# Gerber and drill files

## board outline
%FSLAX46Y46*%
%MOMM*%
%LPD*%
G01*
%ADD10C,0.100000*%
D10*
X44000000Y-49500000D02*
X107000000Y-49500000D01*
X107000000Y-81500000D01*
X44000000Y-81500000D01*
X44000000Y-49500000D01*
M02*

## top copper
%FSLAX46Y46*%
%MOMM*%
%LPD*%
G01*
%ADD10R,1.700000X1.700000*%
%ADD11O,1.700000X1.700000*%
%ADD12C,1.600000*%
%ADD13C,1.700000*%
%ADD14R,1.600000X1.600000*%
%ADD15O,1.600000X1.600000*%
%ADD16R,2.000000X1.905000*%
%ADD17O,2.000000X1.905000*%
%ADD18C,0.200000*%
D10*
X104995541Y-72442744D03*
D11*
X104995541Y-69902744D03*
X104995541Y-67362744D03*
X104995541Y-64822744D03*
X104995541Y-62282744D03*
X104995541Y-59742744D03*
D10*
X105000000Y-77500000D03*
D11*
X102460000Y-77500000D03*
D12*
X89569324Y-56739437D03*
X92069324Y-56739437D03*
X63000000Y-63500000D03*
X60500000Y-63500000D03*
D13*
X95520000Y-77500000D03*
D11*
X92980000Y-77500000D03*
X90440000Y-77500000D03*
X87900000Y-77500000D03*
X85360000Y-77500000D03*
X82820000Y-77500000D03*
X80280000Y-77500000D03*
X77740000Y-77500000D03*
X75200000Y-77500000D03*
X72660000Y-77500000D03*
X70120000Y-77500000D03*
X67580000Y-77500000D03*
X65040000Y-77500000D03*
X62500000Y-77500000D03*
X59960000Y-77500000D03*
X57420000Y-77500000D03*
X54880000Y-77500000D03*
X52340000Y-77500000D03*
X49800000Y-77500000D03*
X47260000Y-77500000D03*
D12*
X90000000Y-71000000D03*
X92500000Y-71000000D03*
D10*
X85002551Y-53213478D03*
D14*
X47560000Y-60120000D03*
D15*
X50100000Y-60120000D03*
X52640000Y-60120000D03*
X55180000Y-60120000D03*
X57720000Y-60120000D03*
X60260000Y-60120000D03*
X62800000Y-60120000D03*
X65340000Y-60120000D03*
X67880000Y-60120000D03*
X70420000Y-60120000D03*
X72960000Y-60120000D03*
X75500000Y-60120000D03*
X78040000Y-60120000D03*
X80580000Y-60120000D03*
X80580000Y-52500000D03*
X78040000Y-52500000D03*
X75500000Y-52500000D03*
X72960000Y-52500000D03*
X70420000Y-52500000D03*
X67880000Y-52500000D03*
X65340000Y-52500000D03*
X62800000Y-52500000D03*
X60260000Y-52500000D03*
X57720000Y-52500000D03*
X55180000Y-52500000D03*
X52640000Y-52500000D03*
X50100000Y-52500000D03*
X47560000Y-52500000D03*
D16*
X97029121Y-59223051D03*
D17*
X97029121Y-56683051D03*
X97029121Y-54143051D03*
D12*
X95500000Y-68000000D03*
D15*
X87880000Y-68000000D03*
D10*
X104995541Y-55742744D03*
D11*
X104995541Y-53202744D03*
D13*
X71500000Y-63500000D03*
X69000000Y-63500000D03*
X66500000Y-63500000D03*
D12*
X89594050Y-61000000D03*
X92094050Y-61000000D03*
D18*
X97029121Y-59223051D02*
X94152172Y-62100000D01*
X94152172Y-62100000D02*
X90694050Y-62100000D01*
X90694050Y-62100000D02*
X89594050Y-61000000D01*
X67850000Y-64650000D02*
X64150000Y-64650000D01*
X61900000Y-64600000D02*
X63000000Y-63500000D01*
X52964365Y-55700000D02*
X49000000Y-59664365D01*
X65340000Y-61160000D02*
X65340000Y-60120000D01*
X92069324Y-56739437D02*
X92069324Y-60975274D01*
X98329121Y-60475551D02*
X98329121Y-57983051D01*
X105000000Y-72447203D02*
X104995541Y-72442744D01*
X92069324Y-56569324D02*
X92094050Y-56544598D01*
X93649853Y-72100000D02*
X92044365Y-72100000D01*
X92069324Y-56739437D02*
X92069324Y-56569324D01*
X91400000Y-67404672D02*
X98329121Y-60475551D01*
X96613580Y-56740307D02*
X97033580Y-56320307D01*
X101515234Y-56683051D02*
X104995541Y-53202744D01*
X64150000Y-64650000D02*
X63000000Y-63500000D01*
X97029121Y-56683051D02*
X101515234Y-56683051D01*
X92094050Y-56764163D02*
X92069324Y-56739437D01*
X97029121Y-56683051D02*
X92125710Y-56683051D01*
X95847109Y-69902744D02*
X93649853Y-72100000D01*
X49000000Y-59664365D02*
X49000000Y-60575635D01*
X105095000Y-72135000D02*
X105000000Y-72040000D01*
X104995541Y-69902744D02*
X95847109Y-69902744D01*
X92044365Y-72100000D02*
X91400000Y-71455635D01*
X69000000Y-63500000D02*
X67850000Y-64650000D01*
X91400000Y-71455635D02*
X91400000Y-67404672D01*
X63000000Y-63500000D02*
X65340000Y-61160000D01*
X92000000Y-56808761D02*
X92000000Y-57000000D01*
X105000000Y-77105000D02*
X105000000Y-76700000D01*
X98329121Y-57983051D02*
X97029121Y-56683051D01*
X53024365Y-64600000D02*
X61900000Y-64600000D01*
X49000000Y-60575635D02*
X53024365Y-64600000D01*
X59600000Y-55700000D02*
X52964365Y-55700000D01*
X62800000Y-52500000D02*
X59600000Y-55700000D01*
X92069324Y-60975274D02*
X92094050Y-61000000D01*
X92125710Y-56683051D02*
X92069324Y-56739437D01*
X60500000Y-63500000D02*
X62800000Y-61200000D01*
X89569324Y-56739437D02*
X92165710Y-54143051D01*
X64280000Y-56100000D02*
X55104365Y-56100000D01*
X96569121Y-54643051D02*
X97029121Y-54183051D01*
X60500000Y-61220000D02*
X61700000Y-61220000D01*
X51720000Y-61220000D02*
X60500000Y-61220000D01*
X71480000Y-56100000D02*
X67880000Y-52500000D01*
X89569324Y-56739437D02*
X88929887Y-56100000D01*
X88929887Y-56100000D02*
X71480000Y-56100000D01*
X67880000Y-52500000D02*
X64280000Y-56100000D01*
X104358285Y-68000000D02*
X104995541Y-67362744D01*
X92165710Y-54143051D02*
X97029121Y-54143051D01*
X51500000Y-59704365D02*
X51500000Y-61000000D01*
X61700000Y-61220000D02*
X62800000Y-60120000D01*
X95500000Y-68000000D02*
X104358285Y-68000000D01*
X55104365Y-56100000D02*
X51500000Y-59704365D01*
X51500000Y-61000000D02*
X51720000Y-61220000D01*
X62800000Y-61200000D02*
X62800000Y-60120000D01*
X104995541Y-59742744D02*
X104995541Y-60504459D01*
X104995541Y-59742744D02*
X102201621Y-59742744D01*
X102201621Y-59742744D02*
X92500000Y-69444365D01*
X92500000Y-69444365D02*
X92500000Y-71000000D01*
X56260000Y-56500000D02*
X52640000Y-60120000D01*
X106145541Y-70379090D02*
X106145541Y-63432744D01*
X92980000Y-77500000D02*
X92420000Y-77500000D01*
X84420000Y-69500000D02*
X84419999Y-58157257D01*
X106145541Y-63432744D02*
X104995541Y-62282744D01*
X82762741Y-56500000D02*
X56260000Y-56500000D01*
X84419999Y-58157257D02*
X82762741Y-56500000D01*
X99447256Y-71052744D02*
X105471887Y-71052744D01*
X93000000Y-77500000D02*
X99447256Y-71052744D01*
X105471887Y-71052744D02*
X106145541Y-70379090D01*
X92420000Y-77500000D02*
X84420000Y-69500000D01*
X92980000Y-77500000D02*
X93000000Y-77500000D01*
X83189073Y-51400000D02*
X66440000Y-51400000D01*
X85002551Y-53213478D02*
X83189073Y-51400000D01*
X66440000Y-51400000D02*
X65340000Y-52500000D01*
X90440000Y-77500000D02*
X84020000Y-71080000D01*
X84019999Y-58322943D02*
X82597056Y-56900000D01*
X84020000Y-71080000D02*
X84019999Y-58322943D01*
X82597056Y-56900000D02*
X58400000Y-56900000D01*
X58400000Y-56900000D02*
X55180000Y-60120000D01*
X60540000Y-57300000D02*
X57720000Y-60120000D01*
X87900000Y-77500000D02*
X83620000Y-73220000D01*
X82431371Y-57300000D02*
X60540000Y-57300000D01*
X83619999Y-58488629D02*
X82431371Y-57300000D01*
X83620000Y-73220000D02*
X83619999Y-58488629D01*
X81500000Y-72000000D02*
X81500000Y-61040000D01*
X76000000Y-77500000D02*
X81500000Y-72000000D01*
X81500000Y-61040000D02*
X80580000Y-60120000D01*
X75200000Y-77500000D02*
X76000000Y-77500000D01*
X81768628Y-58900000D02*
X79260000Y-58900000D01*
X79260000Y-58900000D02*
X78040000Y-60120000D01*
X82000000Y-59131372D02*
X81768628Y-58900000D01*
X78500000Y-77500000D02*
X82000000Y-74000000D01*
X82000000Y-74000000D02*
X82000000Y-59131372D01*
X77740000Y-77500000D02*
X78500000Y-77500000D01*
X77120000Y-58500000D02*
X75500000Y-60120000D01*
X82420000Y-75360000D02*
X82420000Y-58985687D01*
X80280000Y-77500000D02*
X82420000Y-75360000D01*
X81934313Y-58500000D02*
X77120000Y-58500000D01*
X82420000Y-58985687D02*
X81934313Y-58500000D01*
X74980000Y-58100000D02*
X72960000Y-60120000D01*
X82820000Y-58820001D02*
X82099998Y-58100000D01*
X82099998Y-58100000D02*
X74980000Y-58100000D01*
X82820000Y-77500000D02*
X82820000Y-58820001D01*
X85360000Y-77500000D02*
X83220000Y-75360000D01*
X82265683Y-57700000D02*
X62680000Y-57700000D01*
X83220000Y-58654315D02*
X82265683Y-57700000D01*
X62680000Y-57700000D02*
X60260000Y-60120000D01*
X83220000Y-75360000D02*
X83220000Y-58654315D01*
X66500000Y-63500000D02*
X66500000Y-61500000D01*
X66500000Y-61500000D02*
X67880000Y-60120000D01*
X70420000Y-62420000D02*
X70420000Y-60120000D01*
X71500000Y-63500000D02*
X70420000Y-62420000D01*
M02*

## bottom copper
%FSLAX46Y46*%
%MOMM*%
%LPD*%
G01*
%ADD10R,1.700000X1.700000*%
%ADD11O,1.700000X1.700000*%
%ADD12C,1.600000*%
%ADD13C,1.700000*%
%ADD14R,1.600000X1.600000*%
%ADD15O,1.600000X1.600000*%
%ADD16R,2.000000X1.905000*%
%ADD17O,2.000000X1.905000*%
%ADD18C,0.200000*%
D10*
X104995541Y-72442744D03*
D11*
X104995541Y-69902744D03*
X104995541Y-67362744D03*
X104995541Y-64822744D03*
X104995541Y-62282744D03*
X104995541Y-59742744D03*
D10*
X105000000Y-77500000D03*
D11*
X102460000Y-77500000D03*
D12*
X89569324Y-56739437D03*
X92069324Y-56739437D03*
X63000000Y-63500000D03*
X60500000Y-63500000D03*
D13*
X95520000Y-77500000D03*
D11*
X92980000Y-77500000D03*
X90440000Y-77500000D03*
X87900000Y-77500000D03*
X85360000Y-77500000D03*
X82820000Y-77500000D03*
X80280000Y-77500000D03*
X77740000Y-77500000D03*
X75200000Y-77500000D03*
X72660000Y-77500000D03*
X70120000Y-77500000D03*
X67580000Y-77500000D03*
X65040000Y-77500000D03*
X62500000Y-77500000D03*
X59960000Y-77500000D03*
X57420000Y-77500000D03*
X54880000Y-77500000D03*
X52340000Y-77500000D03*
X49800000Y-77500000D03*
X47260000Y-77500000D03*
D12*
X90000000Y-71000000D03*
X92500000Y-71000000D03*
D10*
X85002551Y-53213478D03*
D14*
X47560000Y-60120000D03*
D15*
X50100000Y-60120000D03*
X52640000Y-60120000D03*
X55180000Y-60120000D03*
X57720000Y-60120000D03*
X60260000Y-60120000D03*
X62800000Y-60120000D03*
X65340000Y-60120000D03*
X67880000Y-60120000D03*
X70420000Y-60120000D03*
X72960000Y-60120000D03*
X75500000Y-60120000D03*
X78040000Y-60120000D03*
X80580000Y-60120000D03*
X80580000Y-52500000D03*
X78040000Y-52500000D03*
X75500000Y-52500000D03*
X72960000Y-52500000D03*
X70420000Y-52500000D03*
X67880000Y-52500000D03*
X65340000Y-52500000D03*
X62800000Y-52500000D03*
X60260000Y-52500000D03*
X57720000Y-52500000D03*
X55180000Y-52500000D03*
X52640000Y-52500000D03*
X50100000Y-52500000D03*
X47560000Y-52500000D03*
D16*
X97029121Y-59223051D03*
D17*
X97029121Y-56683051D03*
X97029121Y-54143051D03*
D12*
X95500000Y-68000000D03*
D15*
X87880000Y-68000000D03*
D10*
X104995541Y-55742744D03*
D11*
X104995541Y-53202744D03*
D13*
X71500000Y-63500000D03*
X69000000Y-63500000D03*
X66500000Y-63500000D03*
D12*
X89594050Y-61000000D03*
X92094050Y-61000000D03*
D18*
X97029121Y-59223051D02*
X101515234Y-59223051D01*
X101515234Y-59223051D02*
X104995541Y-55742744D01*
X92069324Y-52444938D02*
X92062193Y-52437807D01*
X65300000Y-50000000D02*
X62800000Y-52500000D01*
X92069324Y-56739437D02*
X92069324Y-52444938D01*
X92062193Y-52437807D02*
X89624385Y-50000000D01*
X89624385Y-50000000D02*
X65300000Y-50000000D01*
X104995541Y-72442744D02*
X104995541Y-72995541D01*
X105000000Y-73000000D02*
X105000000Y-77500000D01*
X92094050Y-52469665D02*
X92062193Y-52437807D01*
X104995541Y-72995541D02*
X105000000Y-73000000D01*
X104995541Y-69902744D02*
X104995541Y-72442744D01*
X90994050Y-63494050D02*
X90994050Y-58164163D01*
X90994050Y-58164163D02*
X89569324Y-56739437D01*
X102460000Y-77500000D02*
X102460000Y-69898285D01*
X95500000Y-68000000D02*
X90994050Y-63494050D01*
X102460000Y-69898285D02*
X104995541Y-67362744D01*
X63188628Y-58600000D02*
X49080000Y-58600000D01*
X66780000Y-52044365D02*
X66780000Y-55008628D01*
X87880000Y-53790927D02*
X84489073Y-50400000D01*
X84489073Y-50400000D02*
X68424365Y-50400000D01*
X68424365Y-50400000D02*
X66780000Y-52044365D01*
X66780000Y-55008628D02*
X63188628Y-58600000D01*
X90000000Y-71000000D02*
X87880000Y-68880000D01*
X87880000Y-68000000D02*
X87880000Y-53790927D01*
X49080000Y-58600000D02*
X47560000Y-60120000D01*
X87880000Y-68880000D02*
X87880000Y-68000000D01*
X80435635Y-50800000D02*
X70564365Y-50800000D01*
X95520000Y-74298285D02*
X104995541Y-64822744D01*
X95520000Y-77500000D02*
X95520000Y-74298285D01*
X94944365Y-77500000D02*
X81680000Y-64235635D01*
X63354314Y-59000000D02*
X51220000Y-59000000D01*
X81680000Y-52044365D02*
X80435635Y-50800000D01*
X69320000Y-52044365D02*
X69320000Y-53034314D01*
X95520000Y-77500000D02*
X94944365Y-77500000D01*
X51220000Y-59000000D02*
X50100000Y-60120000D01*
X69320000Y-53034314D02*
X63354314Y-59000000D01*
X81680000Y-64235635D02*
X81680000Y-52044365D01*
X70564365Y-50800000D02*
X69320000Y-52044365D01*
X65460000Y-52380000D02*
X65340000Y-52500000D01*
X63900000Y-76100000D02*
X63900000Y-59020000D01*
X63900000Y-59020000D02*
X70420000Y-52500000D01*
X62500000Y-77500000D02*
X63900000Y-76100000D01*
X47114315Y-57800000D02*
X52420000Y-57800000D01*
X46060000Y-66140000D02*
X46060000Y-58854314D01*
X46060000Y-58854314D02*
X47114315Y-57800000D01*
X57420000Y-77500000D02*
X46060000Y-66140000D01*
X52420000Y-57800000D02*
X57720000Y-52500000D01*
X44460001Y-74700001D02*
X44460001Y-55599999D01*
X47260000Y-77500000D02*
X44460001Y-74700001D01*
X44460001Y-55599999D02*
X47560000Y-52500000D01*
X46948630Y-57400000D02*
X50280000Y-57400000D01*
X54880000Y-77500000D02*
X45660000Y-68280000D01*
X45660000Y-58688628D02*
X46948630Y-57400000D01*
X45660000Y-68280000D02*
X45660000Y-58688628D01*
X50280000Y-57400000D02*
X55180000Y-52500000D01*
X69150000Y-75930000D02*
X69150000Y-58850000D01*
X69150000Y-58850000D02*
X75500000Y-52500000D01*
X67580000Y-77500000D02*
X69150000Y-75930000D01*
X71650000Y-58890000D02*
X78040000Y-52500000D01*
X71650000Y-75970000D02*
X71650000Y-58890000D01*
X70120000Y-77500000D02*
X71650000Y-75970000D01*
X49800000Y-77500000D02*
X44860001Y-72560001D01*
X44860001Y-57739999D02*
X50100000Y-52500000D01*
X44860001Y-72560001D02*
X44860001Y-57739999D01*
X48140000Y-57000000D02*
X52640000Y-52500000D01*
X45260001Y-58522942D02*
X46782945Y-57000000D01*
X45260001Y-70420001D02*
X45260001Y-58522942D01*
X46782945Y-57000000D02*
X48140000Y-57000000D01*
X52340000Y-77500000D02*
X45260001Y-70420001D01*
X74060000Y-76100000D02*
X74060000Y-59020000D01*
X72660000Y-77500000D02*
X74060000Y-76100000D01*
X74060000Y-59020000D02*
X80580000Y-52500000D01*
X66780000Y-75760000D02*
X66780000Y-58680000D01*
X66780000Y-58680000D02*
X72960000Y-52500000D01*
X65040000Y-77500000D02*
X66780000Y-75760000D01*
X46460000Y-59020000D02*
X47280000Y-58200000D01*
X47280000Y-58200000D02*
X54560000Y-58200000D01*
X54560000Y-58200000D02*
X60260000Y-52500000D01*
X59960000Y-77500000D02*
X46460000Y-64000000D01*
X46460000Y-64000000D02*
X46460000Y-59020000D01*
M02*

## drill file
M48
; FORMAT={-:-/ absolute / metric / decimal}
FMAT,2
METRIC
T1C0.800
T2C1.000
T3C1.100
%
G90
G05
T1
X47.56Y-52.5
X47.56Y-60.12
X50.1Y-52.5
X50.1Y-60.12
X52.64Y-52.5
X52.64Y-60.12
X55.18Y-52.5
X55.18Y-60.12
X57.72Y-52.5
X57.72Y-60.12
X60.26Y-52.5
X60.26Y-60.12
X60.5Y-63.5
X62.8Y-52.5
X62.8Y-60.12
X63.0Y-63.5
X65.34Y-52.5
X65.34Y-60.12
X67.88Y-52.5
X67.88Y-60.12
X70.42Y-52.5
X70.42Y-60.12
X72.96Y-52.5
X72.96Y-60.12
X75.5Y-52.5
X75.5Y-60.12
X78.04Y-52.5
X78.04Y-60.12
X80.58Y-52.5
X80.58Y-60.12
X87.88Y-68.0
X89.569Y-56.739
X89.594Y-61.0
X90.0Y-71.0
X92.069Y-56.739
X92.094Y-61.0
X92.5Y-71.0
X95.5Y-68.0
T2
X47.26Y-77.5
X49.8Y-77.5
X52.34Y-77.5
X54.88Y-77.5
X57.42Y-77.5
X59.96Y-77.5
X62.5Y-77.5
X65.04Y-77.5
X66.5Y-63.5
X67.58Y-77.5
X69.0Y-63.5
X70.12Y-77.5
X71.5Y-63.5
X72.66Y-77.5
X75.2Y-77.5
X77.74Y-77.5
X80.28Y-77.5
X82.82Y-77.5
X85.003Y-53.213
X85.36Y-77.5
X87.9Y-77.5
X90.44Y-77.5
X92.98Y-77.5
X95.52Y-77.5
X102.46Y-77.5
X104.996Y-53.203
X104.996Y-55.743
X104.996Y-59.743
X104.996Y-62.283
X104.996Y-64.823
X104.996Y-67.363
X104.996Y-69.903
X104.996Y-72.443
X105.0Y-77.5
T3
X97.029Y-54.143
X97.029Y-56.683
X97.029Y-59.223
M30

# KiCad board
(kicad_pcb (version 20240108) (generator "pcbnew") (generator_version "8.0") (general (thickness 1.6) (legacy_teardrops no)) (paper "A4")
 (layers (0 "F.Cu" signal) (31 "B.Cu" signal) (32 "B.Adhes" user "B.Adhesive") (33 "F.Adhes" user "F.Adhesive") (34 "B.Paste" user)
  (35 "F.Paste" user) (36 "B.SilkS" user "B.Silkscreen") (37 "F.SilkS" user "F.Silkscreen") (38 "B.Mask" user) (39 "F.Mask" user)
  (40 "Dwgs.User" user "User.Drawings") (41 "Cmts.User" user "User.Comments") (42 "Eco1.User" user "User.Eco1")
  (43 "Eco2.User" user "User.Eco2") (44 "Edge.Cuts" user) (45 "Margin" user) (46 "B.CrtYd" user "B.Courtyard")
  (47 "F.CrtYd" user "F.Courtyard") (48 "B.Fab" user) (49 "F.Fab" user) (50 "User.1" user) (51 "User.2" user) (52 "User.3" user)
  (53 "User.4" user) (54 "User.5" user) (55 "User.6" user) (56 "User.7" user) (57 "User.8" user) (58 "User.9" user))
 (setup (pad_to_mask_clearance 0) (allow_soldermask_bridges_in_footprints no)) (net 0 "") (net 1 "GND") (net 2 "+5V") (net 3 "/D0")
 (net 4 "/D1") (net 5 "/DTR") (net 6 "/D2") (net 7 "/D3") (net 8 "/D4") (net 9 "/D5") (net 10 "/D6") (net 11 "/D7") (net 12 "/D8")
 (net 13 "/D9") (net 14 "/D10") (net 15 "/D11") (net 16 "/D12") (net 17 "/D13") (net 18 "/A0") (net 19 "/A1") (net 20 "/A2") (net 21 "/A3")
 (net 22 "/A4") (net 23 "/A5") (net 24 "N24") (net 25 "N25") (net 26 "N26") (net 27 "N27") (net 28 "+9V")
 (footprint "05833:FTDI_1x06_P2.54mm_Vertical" (layer "F.Cu") (at 104.995541 72.442744 180)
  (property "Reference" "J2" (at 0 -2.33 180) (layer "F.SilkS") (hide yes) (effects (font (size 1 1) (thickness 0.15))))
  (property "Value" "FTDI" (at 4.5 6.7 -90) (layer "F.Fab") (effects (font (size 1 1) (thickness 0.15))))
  (pad "1" thru_hole rect (at 0 0 180) (size 1.7 1.7) (drill 1) (layers "*.Cu" "*.Mask") (remove_unused_layers no) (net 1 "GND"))
  (pad "2" thru_hole oval (at 0 2.54 180) (size 1.7 1.7) (drill 1) (layers "*.Cu" "*.Mask") (remove_unused_layers no) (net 1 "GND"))
  (pad "3" thru_hole oval (at 0 5.08 180) (size 1.7 1.7) (drill 1) (layers "*.Cu" "*.Mask") (remove_unused_layers no) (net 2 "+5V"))
  (pad "4" thru_hole oval (at 0 7.62 180) (size 1.7 1.7) (drill 1) (layers "*.Cu" "*.Mask") (remove_unused_layers no) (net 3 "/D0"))
  (pad "5" thru_hole oval (at 0 10.16 180) (size 1.7 1.7) (drill 1) (layers "*.Cu" "*.Mask") (remove_unused_layers no) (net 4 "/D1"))
  (pad "6" thru_hole oval (at 0 12.7 180) (size 1.7 1.7) (drill 1) (layers "*.Cu" "*.Mask") (remove_unused_layers no) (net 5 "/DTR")))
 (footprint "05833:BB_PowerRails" (layer "F.Cu") (at 105 77.5 -90)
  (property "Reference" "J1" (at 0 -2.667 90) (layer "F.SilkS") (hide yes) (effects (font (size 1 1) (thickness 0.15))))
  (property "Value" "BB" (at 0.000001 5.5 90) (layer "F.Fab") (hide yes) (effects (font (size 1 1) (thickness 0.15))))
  (pad "1" thru_hole rect (at 0 0 270) (size 1.7 1.7) (drill 1) (layers "*.Cu" "*.Mask") (remove_unused_layers no) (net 1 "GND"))
  (pad "2" thru_hole oval (at 0 2.54 270) (size 1.7 1.7) (drill 1) (layers "*.Cu" "*.Mask") (remove_unused_layers no) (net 2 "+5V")))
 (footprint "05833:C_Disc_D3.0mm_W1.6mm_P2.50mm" (layer "F.Cu") (at 89.569324 56.739437)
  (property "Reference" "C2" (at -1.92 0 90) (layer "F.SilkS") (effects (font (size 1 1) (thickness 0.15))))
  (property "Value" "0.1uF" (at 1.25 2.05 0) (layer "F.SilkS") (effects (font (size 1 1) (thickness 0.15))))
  (pad "1" thru_hole circle (at 0 0) (size 1.6 1.6) (drill 0.8) (layers "*.Cu" "*.Mask") (remove_unused_layers no) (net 2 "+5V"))
  (pad "2" thru_hole circle (at 2.5 0) (size 1.6 1.6) (drill 0.8) (layers "*.Cu" "*.Mask") (remove_unused_layers no) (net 1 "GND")))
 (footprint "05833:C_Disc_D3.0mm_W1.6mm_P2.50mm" (layer "F.Cu") (at 63 63.5 180)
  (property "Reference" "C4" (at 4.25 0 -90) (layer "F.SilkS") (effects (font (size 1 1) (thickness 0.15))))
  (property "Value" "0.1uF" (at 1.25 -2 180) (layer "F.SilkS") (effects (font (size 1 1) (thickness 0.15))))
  (pad "1" thru_hole circle (at 0 0 180) (size 1.6 1.6) (drill 0.8) (layers "*.Cu" "*.Mask") (remove_unused_layers no) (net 1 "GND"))
  (pad "2" thru_hole circle (at 2.5 0 180) (size 1.6 1.6) (drill 0.8) (layers "*.Cu" "*.Mask") (remove_unused_layers no) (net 2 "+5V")))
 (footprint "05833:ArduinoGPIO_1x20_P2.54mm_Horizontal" (layer "F.Cu") (at 95.52 77.5 -90)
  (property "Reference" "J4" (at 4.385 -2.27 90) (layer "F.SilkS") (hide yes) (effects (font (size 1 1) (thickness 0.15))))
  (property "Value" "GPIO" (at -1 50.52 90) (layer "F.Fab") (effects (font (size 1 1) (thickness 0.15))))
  (pad "1" thru_hole circle (at 0 0 270) (size 1.7 1.7) (drill 1) (layers "*.Cu" "*.Mask") (remove_unused_layers no) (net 3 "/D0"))
  (pad "2" thru_hole oval (at 0 2.54 270) (size 1.7 1.7) (drill 1) (layers "*.Cu" "*.Mask") (remove_unused_layers no) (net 4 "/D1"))
  (pad "3" thru_hole oval (at 0 5.08 270) (size 1.7 1.7) (drill 1) (layers "*.Cu" "*.Mask") (remove_unused_layers no) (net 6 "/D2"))
  (pad "4" thru_hole oval (at 0 7.62 270) (size 1.7 1.7) (drill 1) (layers "*.Cu" "*.Mask") (remove_unused_layers no) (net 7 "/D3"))
  (pad "5" thru_hole oval (at 0 10.16 270) (size 1.7 1.7) (drill 1) (layers "*.Cu" "*.Mask") (remove_unused_layers no) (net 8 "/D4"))
  (pad "6" thru_hole oval (at 0 12.7 270) (size 1.7 1.7) (drill 1) (layers "*.Cu" "*.Mask") (remove_unused_layers no) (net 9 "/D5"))
  (pad "7" thru_hole oval (at 0 15.24 270) (size 1.7 1.7) (drill 1) (layers "*.Cu" "*.Mask") (remove_unused_layers no) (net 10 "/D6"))
  (pad "8" thru_hole oval (at 0 17.78 270) (size 1.7 1.7) (drill 1) (layers "*.Cu" "*.Mask") (remove_unused_layers no) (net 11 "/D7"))
  (pad "9" thru_hole oval (at 0 20.32 270) (size 1.7 1.7) (drill 1) (layers "*.Cu" "*.Mask") (remove_unused_layers no) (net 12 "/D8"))
  (pad "10" thru_hole oval (at 0 22.86 270) (size 1.7 1.7) (drill 1) (layers "*.Cu" "*.Mask") (remove_unused_layers no) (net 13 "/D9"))
  (pad "11" thru_hole oval (at 0 25.4 270) (size 1.7 1.7) (drill 1) (layers "*.Cu" "*.Mask") (remove_unused_layers no) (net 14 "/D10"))
  (pad "12" thru_hole oval (at 0 27.94 270) (size 1.7 1.7) (drill 1) (layers "*.Cu" "*.Mask") (remove_unused_layers no) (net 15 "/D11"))
  (pad "13" thru_hole oval (at 0 30.48 270) (size 1.7 1.7) (drill 1) (layers "*.Cu" "*.Mask") (remove_unused_layers no) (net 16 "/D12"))
  (pad "14" thru_hole oval (at 0 33.02 270) (size 1.7 1.7) (drill 1) (layers "*.Cu" "*.Mask") (remove_unused_layers no) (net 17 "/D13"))
  (pad "15" thru_hole oval (at 0 35.56 270) (size 1.7 1.7) (drill 1) (layers "*.Cu" "*.Mask") (remove_unused_layers no) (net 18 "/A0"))
  (pad "16" thru_hole oval (at 0 38.1 270) (size 1.7 1.7) (drill 1) (layers "*.Cu" "*.Mask") (remove_unused_layers no) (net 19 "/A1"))
  (pad "17" thru_hole oval (at 0 40.64 270) (size 1.7 1.7) (drill 1) (layers "*.Cu" "*.Mask") (remove_unused_layers no) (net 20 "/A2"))
  (pad "18" thru_hole oval (at 0 43.18 270) (size 1.7 1.7) (drill 1) (layers "*.Cu" "*.Mask") (remove_unused_layers no) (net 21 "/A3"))
  (pad "19" thru_hole oval (at 0 45.72 270) (size 1.7 1.7) (drill 1) (layers "*.Cu" "*.Mask") (remove_unused_layers no) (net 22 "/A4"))
  (pad "20" thru_hole oval (at 0 48.26 270) (size 1.7 1.7) (drill 1) (layers "*.Cu" "*.Mask") (remove_unused_layers no) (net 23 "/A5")))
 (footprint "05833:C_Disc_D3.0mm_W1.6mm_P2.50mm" (layer "F.Cu") (at 90 71)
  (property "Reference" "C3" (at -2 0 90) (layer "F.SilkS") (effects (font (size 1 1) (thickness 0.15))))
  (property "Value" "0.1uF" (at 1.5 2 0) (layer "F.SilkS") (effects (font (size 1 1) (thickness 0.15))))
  (pad "1" thru_hole circle (at 0 0) (size 1.6 1.6) (drill 0.8) (layers "*.Cu" "*.Mask") (remove_unused_layers no) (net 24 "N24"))
  (pad "2" thru_hole circle (at 2.5 0) (size 1.6 1.6) (drill 0.8) (layers "*.Cu" "*.Mask") (remove_unused_layers no) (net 5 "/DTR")))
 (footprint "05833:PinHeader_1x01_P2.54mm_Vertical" (layer "F.Cu") (at 85.002551 53.213478)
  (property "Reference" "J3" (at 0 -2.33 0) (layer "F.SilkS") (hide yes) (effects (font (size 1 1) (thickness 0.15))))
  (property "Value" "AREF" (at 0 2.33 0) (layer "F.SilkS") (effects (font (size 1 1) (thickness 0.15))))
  (pad "1" thru_hole rect (at 0 0) (size 1.7 1.7) (drill 1) (layers "*.Cu" "*.Mask") (remove_unused_layers no) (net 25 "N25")))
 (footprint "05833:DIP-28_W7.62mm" (layer "F.Cu") (at 47.56 60.12 90)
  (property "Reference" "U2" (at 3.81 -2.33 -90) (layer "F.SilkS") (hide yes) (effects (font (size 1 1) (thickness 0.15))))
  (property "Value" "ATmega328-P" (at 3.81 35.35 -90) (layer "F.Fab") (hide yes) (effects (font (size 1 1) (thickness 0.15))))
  (pad "1" thru_hole rect (at 0 0 90) (size 1.6 1.6) (drill 0.8) (layers "*.Cu" "*.Mask") (remove_unused_layers no) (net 24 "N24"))
  (pad "2" thru_hole oval (at 0 2.54 90) (size 1.6 1.6) (drill 0.8) (layers "*.Cu" "*.Mask") (remove_unused_layers no) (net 3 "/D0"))
  (pad "3" thru_hole oval (at 0 5.08 90) (size 1.6 1.6) (drill 0.8) (layers "*.Cu" "*.Mask") (remove_unused_layers no) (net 4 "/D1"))
  (pad "4" thru_hole oval (at 0 7.62 90) (size 1.6 1.6) (drill 0.8) (layers "*.Cu" "*.Mask") (remove_unused_layers no) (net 6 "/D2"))
  (pad "5" thru_hole oval (at 0 10.16 90) (size 1.6 1.6) (drill 0.8) (layers "*.Cu" "*.Mask") (remove_unused_layers no) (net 7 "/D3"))
  (pad "6" thru_hole oval (at 0 12.7 90) (size 1.6 1.6) (drill 0.8) (layers "*.Cu" "*.Mask") (remove_unused_layers no) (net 8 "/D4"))
  (pad "7" thru_hole oval (at 0 15.24 90) (size 1.6 1.6) (drill 0.8) (layers "*.Cu" "*.Mask") (remove_unused_layers no) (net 2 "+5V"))
  (pad "8" thru_hole oval (at 0 17.78 90) (size 1.6 1.6) (drill 0.8) (layers "*.Cu" "*.Mask") (remove_unused_layers no) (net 1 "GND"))
  (pad "9" thru_hole oval (at 0 20.32 90) (size 1.6 1.6) (drill 0.8) (layers "*.Cu" "*.Mask") (remove_unused_layers no) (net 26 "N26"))
  (pad "10" thru_hole oval (at 0 22.86 90) (size 1.6 1.6) (drill 0.8) (layers "*.Cu" "*.Mask") (remove_unused_layers no) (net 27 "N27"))
  (pad "11" thru_hole oval (at 0 25.4 90) (size 1.6 1.6) (drill 0.8) (layers "*.Cu" "*.Mask") (remove_unused_layers no) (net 9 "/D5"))
  (pad "12" thru_hole oval (at 0 27.94 90) (size 1.6 1.6) (drill 0.8) (layers "*.Cu" "*.Mask") (remove_unused_layers no) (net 10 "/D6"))
  (pad "13" thru_hole oval (at 0 30.48 90) (size 1.6 1.6) (drill 0.8) (layers "*.Cu" "*.Mask") (remove_unused_layers no) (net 11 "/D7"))
  (pad "14" thru_hole oval (at 0 33.02 90) (size 1.6 1.6) (drill 0.8) (layers "*.Cu" "*.Mask") (remove_unused_layers no) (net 12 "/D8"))
  (pad "15" thru_hole oval (at 7.62 33.02 90) (size 1.6 1.6) (drill 0.8) (layers "*.Cu" "*.Mask") (remove_unused_layers no) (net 13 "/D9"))
  (pad "16" thru_hole oval (at 7.62 30.48 90) (size 1.6 1.6) (drill 0.8) (layers "*.Cu" "*.Mask") (remove_unused_layers no) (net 14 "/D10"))
  (pad "17" thru_hole oval (at 7.62 27.94 90) (size 1.6 1.6) (drill 0.8) (layers "*.Cu" "*.Mask") (remove_unused_layers no) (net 15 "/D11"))
  (pad "18" thru_hole oval (at 7.62 25.4 90) (size 1.6 1.6) (drill 0.8) (layers "*.Cu" "*.Mask") (remove_unused_layers no) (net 16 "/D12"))
  (pad "19" thru_hole oval (at 7.62 22.86 90) (size 1.6 1.6) (drill 0.8) (layers "*.Cu" "*.Mask") (remove_unused_layers no) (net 17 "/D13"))
  (pad "20" thru_hole oval (at 7.62 20.32 90) (size 1.6 1.6) (drill 0.8) (layers "*.Cu" "*.Mask") (remove_unused_layers no) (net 2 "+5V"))
  (pad "21" thru_hole oval (at 7.62 17.78 90) (size 1.6 1.6) (drill 0.8) (layers "*.Cu" "*.Mask") (remove_unused_layers no) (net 25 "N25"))
  (pad "22" thru_hole oval (at 7.62 15.24 90) (size 1.6 1.6) (drill 0.8) (layers "*.Cu" "*.Mask") (remove_unused_layers no) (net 1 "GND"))
  (pad "23" thru_hole oval (at 7.62 12.7 90) (size 1.6 1.6) (drill 0.8) (layers "*.Cu" "*.Mask") (remove_unused_layers no) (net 18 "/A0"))
  (pad "24" thru_hole oval (at 7.62 10.16 90) (size 1.6 1.6) (drill 0.8) (layers "*.Cu" "*.Mask") (remove_unused_layers no) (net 19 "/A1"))
  (pad "25" thru_hole oval (at 7.62 7.62 90) (size 1.6 1.6) (drill 0.8) (layers "*.Cu" "*.Mask") (remove_unused_layers no) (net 20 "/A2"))
  (pad "26" thru_hole oval (at 7.62 5.08 90) (size 1.6 1.6) (drill 0.8) (layers "*.Cu" "*.Mask") (remove_unused_layers no) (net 21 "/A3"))
  (pad "27" thru_hole oval (at 7.62 2.54 90) (size 1.6 1.6) (drill 0.8) (layers "*.Cu" "*.Mask") (remove_unused_layers no) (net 22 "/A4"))
  (pad "28" thru_hole oval (at 7.62 0 90) (size 1.6 1.6) (drill 0.8) (layers "*.Cu" "*.Mask") (remove_unused_layers no) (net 23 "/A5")))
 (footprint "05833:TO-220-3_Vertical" (layer "F.Cu") (at 97.029121 59.223051 90)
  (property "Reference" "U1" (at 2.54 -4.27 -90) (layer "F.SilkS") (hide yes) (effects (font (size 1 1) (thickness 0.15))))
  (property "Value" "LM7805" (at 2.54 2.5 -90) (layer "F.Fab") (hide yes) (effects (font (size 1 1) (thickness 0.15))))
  (pad "1" thru_hole rect (at 0 0 90) (size 1.905 2) (drill 1.1) (layers "*.Cu" "*.Mask") (remove_unused_layers no) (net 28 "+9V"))
  (pad "2" thru_hole oval (at 2.54 0 90) (size 1.905 2) (drill 1.1) (layers "*.Cu" "*.Mask") (remove_unused_layers no) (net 1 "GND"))
  (pad "3" thru_hole oval (at 5.08 0 90) (size 1.905 2) (drill 1.1) (layers "*.Cu" "*.Mask") (remove_unused_layers no) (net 2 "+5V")))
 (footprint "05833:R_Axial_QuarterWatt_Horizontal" (layer "F.Cu") (at 95.5 68 180)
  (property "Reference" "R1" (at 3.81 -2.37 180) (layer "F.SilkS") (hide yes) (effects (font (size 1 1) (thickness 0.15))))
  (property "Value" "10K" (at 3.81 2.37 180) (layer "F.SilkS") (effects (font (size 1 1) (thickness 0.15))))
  (pad "1" thru_hole circle (at 0 0 180) (size 1.6 1.6) (drill 0.8) (layers "*.Cu" "*.Mask") (remove_unused_layers no) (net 2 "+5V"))
  (pad "2" thru_hole oval (at 7.62 0 180) (size 1.6 1.6) (drill 0.8) (layers "*.Cu" "*.Mask") (remove_unused_layers no) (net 24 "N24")))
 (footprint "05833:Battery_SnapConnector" (layer "F.Cu") (at 104.995541 55.742744 180)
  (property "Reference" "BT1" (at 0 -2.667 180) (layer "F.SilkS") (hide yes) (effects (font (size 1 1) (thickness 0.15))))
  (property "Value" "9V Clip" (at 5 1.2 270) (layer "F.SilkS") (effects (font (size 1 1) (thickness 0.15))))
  (pad "1" thru_hole rect (at 0 0 180) (size 1.7 1.7) (drill 1) (layers "*.Cu" "*.Mask") (remove_unused_layers no) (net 28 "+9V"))
  (pad "2" thru_hole oval (at 0 2.54 180) (size 1.7 1.7) (drill 1) (layers "*.Cu" "*.Mask") (remove_unused_layers no) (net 1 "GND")))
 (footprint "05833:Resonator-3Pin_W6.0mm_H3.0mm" (layer "F.Cu") (at 71.5 63.5 180)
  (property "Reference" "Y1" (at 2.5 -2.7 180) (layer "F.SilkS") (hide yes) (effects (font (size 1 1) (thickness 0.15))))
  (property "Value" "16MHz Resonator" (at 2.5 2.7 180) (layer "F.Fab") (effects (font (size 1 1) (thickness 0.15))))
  (pad "1" thru_hole circle (at 0 0 180) (size 1.7 1.7) (drill 1) (layers "*.Cu" "*.Mask") (remove_unused_layers no) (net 27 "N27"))
  (pad "2" thru_hole circle (at 2.5 0 180) (size 1.7 1.7) (drill 1) (layers "*.Cu" "*.Mask") (remove_unused_layers no) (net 1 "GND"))
  (pad "3" thru_hole circle (at 5 0 180) (size 1.7 1.7) (drill 1) (layers "*.Cu" "*.Mask") (remove_unused_layers no) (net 26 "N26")))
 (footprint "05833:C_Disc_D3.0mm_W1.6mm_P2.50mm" (layer "F.Cu") (at 89.59405 61)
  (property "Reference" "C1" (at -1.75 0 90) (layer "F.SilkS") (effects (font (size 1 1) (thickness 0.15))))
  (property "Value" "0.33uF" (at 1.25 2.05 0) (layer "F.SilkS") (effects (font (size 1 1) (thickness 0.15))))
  (pad "1" thru_hole circle (at 0 0) (size 1.6 1.6) (drill 0.8) (layers "*.Cu" "*.Mask") (remove_unused_layers no) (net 28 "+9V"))
  (pad "2" thru_hole circle (at 2.5 0) (size 1.6 1.6) (drill 0.8) (layers "*.Cu" "*.Mask") (remove_unused_layers no) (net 1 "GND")))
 (gr_rect (start 44 49.5) (end 107 81.5) (stroke (width 0.1) (type default)) (fill none) (layer "Edge.Cuts"))
 (segment (start 97.029121 59.223051) (end 94.152172 62.1) (width 0.2) (layer "F.Cu") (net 28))
 (segment (start 94.152172 62.1) (end 90.69405 62.1) (width 0.2) (layer "F.Cu") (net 28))
 (segment (start 90.69405 62.1) (end 89.59405 61) (width 0.2) (layer "F.Cu") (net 28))
 (segment (start 97.029121 59.223051) (end 101.515234 59.223051) (width 0.2) (layer "B.Cu") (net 28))
 (segment (start 101.515234 59.223051) (end 104.995541 55.742744) (width 0.2) (layer "B.Cu") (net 28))
 (segment (start 67.85 64.65) (end 64.15 64.65) (width 0.2) (layer "F.Cu") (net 1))
 (segment (start 61.9 64.6) (end 63 63.5) (width 0.2) (layer "F.Cu") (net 1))
 (segment (start 52.964365 55.7) (end 49 59.664365) (width 0.2) (layer "F.Cu") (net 1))
 (segment (start 65.34 61.16) (end 65.34 60.12) (width 0.2) (layer "F.Cu") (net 1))
 (segment (start 92.069324 56.739437) (end 92.069324 60.975274) (width 0.2) (layer "F.Cu") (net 1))
 (segment (start 98.329121 60.475551) (end 98.329121 57.983051) (width 0.2) (layer "F.Cu") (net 1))
 (segment (start 105 72.447203) (end 104.995541 72.442744) (width 0.2) (layer "F.Cu") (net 1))
 (segment (start 92.069324 56.569324) (end 92.09405 56.544598) (width 0.2) (layer "F.Cu") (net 1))
 (segment (start 93.649853 72.1) (end 92.044365 72.1) (width 0.2) (layer "F.Cu") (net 1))
 (segment (start 92.069324 56.739437) (end 92.069324 56.569324) (width 0.2) (layer "F.Cu") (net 1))
 (segment (start 91.4 67.404672) (end 98.329121 60.475551) (width 0.2) (layer "F.Cu") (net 1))
 (segment (start 96.61358 56.740307) (end 97.03358 56.320307) (width 0.2) (layer "F.Cu") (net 1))
 (segment (start 101.515234 56.683051) (end 104.995541 53.202744) (width 0.2) (layer "F.Cu") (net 1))
 (segment (start 64.15 64.65) (end 63 63.5) (width 0.2) (layer "F.Cu") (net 1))
 (segment (start 97.029121 56.683051) (end 101.515234 56.683051) (width 0.2) (layer "F.Cu") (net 1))
 (segment (start 92.09405 56.764163) (end 92.069324 56.739437) (width 0.2) (layer "F.Cu") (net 1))
 (segment (start 97.029121 56.683051) (end 92.12571 56.683051) (width 0.2) (layer "F.Cu") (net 1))
 (segment (start 95.847109 69.902744) (end 93.649853 72.1) (width 0.2) (layer "F.Cu") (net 1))
 (segment (start 49 59.664365) (end 49 60.575635) (width 0.2) (layer "F.Cu") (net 1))
 (segment (start 105.095 72.135) (end 105 72.04) (width 0.2) (layer "F.Cu") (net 1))
 (segment (start 104.995541 69.902744) (end 95.847109 69.902744) (width 0.2) (layer "F.Cu") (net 1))
 (segment (start 92.044365 72.1) (end 91.4 71.455635) (width 0.2) (layer "F.Cu") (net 1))
 (segment (start 69 63.5) (end 67.85 64.65) (width 0.2) (layer "F.Cu") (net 1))
 (segment (start 91.4 71.455635) (end 91.4 67.404672) (width 0.2) (layer "F.Cu") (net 1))
 (segment (start 63 63.5) (end 65.34 61.16) (width 0.2) (layer "F.Cu") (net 1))
 (segment (start 92 56.808761) (end 92 57) (width 0.2) (layer "F.Cu") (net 1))
 (segment (start 105 77.105) (end 105 76.7) (width 0.2) (layer "F.Cu") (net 1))
 (segment (start 98.329121 57.983051) (end 97.029121 56.683051) (width 0.2) (layer "F.Cu") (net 1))
 (segment (start 53.024365 64.6) (end 61.9 64.6) (width 0.2) (layer "F.Cu") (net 1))
 (segment (start 49 60.575635) (end 53.024365 64.6) (width 0.2) (layer "F.Cu") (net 1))
 (segment (start 59.6 55.7) (end 52.964365 55.7) (width 0.2) (layer "F.Cu") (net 1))
 (segment (start 62.8 52.5) (end 59.6 55.7) (width 0.2) (layer "F.Cu") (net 1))
 (segment (start 92.069324 60.975274) (end 92.09405 61) (width 0.2) (layer "F.Cu") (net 1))
 (segment (start 92.12571 56.683051) (end 92.069324 56.739437) (width 0.2) (layer "F.Cu") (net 1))
 (segment (start 92.069324 52.444938) (end 92.062193 52.437807) (width 0.2) (layer "B.Cu") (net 1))
 (segment (start 65.3 50) (end 62.8 52.5) (width 0.2) (layer "B.Cu") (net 1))
 (segment (start 92.069324 56.739437) (end 92.069324 52.444938) (width 0.2) (layer "B.Cu") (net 1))
 (segment (start 92.062193 52.437807) (end 89.624385 50) (width 0.2) (layer "B.Cu") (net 1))
 (segment (start 89.624385 50) (end 65.3 50) (width 0.2) (layer "B.Cu") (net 1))
 (segment (start 104.995541 72.442744) (end 104.995541 72.995541) (width 0.2) (layer "B.Cu") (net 1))
 (segment (start 105 73) (end 105 77.5) (width 0.2) (layer "B.Cu") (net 1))
 (segment (start 92.09405 52.469665) (end 92.062193 52.437807) (width 0.2) (layer "B.Cu") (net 1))
 (segment (start 104.995541 72.995541) (end 105 73) (width 0.2) (layer "B.Cu") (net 1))
 (segment (start 104.995541 69.902744) (end 104.995541 72.442744) (width 0.2) (layer "B.Cu") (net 1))
 (segment (start 60.5 63.5) (end 62.8 61.2) (width 0.2) (layer "F.Cu") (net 2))
 (segment (start 89.569324 56.739437) (end 92.16571 54.143051) (width 0.2) (layer "F.Cu") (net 2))
 (segment (start 64.28 56.1) (end 55.104365 56.1) (width 0.2) (layer "F.Cu") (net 2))
 (segment (start 96.569121 54.643051) (end 97.029121 54.183051) (width 0.2) (layer "F.Cu") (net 2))
 (segment (start 60.5 61.22) (end 61.7 61.22) (width 0.2) (layer "F.Cu") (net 2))
 (segment (start 51.72 61.22) (end 60.5 61.22) (width 0.2) (layer "F.Cu") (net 2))
 (segment (start 71.48 56.1) (end 67.88 52.5) (width 0.2) (layer "F.Cu") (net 2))
 (segment (start 89.569324 56.739437) (end 88.929887 56.1) (width 0.2) (layer "F.Cu") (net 2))
 (segment (start 88.929887 56.1) (end 71.48 56.1) (width 0.2) (layer "F.Cu") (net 2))
 (segment (start 67.88 52.5) (end 64.28 56.1) (width 0.2) (layer "F.Cu") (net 2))
 (segment (start 104.358285 68) (end 104.995541 67.362744) (width 0.2) (layer "F.Cu") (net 2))
 (segment (start 92.16571 54.143051) (end 97.029121 54.143051) (width 0.2) (layer "F.Cu") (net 2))
 (segment (start 51.5 59.704365) (end 51.5 61) (width 0.2) (layer "F.Cu") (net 2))
 (segment (start 61.7 61.22) (end 62.8 60.12) (width 0.2) (layer "F.Cu") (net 2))
 (segment (start 95.5 68) (end 104.358285 68) (width 0.2) (layer "F.Cu") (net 2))
 (segment (start 55.104365 56.1) (end 51.5 59.704365) (width 0.2) (layer "F.Cu") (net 2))
 (segment (start 51.5 61) (end 51.72 61.22) (width 0.2) (layer "F.Cu") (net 2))
 (segment (start 62.8 61.2) (end 62.8 60.12) (width 0.2) (layer "F.Cu") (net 2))
 (segment (start 90.99405 63.49405) (end 90.99405 58.164163) (width 0.2) (layer "B.Cu") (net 2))
 (segment (start 90.99405 58.164163) (end 89.569324 56.739437) (width 0.2) (layer "B.Cu") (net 2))
 (segment (start 102.46 77.5) (end 102.46 69.898285) (width 0.2) (layer "B.Cu") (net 2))
 (segment (start 95.5 68) (end 90.99405 63.49405) (width 0.2) (layer "B.Cu") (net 2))
 (segment (start 102.46 69.898285) (end 104.995541 67.362744) (width 0.2) (layer "B.Cu") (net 2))
 (segment (start 104.995541 59.742744) (end 104.995541 60.504459) (width 0.2) (layer "F.Cu") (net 5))
 (segment (start 104.995541 59.742744) (end 102.201621 59.742744) (width 0.2) (layer "F.Cu") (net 5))
 (segment (start 102.201621 59.742744) (end 92.5 69.444365) (width 0.2) (layer "F.Cu") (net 5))
 (segment (start 92.5 69.444365) (end 92.5 71) (width 0.2) (layer "F.Cu") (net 5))
 (segment (start 63.188628 58.6) (end 49.08 58.6) (width 0.2) (layer "B.Cu") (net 24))
 (segment (start 66.78 52.044365) (end 66.78 55.008628) (width 0.2) (layer "B.Cu") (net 24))
 (segment (start 87.88 53.790927) (end 84.489073 50.4) (width 0.2) (layer "B.Cu") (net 24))
 (segment (start 84.489073 50.4) (end 68.424365 50.4) (width 0.2) (layer "B.Cu") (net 24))
 (segment (start 68.424365 50.4) (end 66.78 52.044365) (width 0.2) (layer "B.Cu") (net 24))
 (segment (start 66.78 55.008628) (end 63.188628 58.6) (width 0.2) (layer "B.Cu") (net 24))
 (segment (start 90 71) (end 87.88 68.88) (width 0.2) (layer "B.Cu") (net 24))
 (segment (start 87.88 68) (end 87.88 53.790927) (width 0.2) (layer "B.Cu") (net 24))
 (segment (start 49.08 58.6) (end 47.56 60.12) (width 0.2) (layer "B.Cu") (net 24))
 (segment (start 87.88 68.88) (end 87.88 68) (width 0.2) (layer "B.Cu") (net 24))
 (segment (start 56.26 56.5) (end 52.64 60.12) (width 0.2) (layer "F.Cu") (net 4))
 (segment (start 106.145541 70.37909) (end 106.145541 63.432744) (width 0.2) (layer "F.Cu") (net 4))
 (segment (start 92.98 77.5) (end 92.42 77.5) (width 0.2) (layer "F.Cu") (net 4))
 (segment (start 84.42 69.5) (end 84.419999 58.157257) (width 0.2) (layer "F.Cu") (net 4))
 (segment (start 106.145541 63.432744) (end 104.995541 62.282744) (width 0.2) (layer "F.Cu") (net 4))
 (segment (start 82.762741 56.5) (end 56.26 56.5) (width 0.2) (layer "F.Cu") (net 4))
 (segment (start 84.419999 58.157257) (end 82.762741 56.5) (width 0.2) (layer "F.Cu") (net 4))
 (segment (start 99.447256 71.052744) (end 105.471887 71.052744) (width 0.2) (layer "F.Cu") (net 4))
 (segment (start 93 77.5) (end 99.447256 71.052744) (width 0.2) (layer "F.Cu") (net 4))
 (segment (start 105.471887 71.052744) (end 106.145541 70.37909) (width 0.2) (layer "F.Cu") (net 4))
 (segment (start 92.42 77.5) (end 84.42 69.5) (width 0.2) (layer "F.Cu") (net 4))
 (segment (start 92.98 77.5) (end 93 77.5) (width 0.2) (layer "F.Cu") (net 4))
 (segment (start 80.435635 50.8) (end 70.564365 50.8) (width 0.2) (layer "B.Cu") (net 3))
 (segment (start 95.52 74.298285) (end 104.995541 64.822744) (width 0.2) (layer "B.Cu") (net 3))
 (segment (start 95.52 77.5) (end 95.52 74.298285) (width 0.2) (layer "B.Cu") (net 3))
 (segment (start 94.944365 77.5) (end 81.68 64.235635) (width 0.2) (layer "B.Cu") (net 3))
 (segment (start 63.354314 59) (end 51.22 59) (width 0.2) (layer "B.Cu") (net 3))
 (segment (start 81.68 52.044365) (end 80.435635 50.8) (width 0.2) (layer "B.Cu") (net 3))
 (segment (start 69.32 52.044365) (end 69.32 53.034314) (width 0.2) (layer "B.Cu") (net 3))
 (segment (start 95.52 77.5) (end 94.944365 77.5) (width 0.2) (layer "B.Cu") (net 3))
 (segment (start 51.22 59) (end 50.1 60.12) (width 0.2) (layer "B.Cu") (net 3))
 (segment (start 69.32 53.034314) (end 63.354314 59) (width 0.2) (layer "B.Cu") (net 3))
 (segment (start 81.68 64.235635) (end 81.68 52.044365) (width 0.2) (layer "B.Cu") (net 3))
 (segment (start 70.564365 50.8) (end 69.32 52.044365) (width 0.2) (layer "B.Cu") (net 3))
 (segment (start 83.189073 51.4) (end 66.44 51.4) (width 0.2) (layer "F.Cu") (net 25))
 (segment (start 85.002551 53.213478) (end 83.189073 51.4) (width 0.2) (layer "F.Cu") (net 25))
 (segment (start 66.44 51.4) (end 65.34 52.5) (width 0.2) (layer "F.Cu") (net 25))
 (segment (start 65.46 52.38) (end 65.34 52.5) (width 0.2) (layer "B.Cu") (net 25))
 (segment (start 63.9 76.1) (end 63.9 59.02) (width 0.2) (layer "B.Cu") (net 17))
 (segment (start 63.9 59.02) (end 70.42 52.5) (width 0.2) (layer "B.Cu") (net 17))
 (segment (start 62.5 77.5) (end 63.9 76.1) (width 0.2) (layer "B.Cu") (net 17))
 (segment (start 47.114315 57.8) (end 52.42 57.8) (width 0.2) (layer "B.Cu") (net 19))
 (segment (start 46.06 66.14) (end 46.06 58.854314) (width 0.2) (layer "B.Cu") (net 19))
 (segment (start 46.06 58.854314) (end 47.114315 57.8) (width 0.2) (layer "B.Cu") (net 19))
 (segment (start 57.42 77.5) (end 46.06 66.14) (width 0.2) (layer "B.Cu") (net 19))
 (segment (start 52.42 57.8) (end 57.72 52.5) (width 0.2) (layer "B.Cu") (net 19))
 (segment (start 90.44 77.5) (end 84.02 71.08) (width 0.2) (layer "F.Cu") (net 6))
 (segment (start 84.019999 58.322943) (end 82.597056 56.9) (width 0.2) (layer "F.Cu") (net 6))
 (segment (start 84.02 71.08) (end 84.019999 58.322943) (width 0.2) (layer "F.Cu") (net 6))
 (segment (start 82.597056 56.9) (end 58.4 56.9) (width 0.2) (layer "F.Cu") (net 6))
 (segment (start 58.4 56.9) (end 55.18 60.12) (width 0.2) (layer "F.Cu") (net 6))
 (segment (start 44.460001 74.700001) (end 44.460001 55.599999) (width 0.2) (layer "B.Cu") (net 23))
 (segment (start 47.26 77.5) (end 44.460001 74.700001) (width 0.2) (layer "B.Cu") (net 23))
 (segment (start 44.460001 55.599999) (end 47.56 52.5) (width 0.2) (layer "B.Cu") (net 23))
 (segment (start 46.94863 57.4) (end 50.28 57.4) (width 0.2) (layer "B.Cu") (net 20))
 (segment (start 54.88 77.5) (end 45.66 68.28) (width 0.2) (layer "B.Cu") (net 20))
 (segment (start 45.66 58.688628) (end 46.94863 57.4) (width 0.2) (layer "B.Cu") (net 20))
 (segment (start 45.66 68.28) (end 45.66 58.688628) (width 0.2) (layer "B.Cu") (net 20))
 (segment (start 50.28 57.4) (end 55.18 52.5) (width 0.2) (layer "B.Cu") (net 20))
 (segment (start 60.54 57.3) (end 57.72 60.12) (width 0.2) (layer "F.Cu") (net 7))
 (segment (start 87.9 77.5) (end 83.62 73.22) (width 0.2) (layer "F.Cu") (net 7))
 (segment (start 82.431371 57.3) (end 60.54 57.3) (width 0.2) (layer "F.Cu") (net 7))
 (segment (start 83.619999 58.488629) (end 82.431371 57.3) (width 0.2) (layer "F.Cu") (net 7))
 (segment (start 83.62 73.22) (end 83.619999 58.488629) (width 0.2) (layer "F.Cu") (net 7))
 (segment (start 69.15 75.93) (end 69.15 58.85) (width 0.2) (layer "B.Cu") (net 15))
 (segment (start 69.15 58.85) (end 75.5 52.5) (width 0.2) (layer "B.Cu") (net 15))
 (segment (start 67.58 77.5) (end 69.15 75.93) (width 0.2) (layer "B.Cu") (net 15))
 (segment (start 81.5 72) (end 81.5 61.04) (width 0.2) (layer "F.Cu") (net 12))
 (segment (start 76 77.5) (end 81.5 72) (width 0.2) (layer "F.Cu") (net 12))
 (segment (start 81.5 61.04) (end 80.58 60.12) (width 0.2) (layer "F.Cu") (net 12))
 (segment (start 75.2 77.5) (end 76 77.5) (width 0.2) (layer "F.Cu") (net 12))
 (segment (start 71.65 58.89) (end 78.04 52.5) (width 0.2) (layer "B.Cu") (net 14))
 (segment (start 71.65 75.97) (end 71.65 58.89) (width 0.2) (layer "B.Cu") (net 14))
 (segment (start 70.12 77.5) (end 71.65 75.97) (width 0.2) (layer "B.Cu") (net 14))
 (segment (start 81.768628 58.9) (end 79.26 58.9) (width 0.2) (layer "F.Cu") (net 11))
 (segment (start 79.26 58.9) (end 78.04 60.12) (width 0.2) (layer "F.Cu") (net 11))
 (segment (start 82 59.131372) (end 81.768628 58.9) (width 0.2) (layer "F.Cu") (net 11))
 (segment (start 78.5 77.5) (end 82 74) (width 0.2) (layer "F.Cu") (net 11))
 (segment (start 82 74) (end 82 59.131372) (width 0.2) (layer "F.Cu") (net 11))
 (segment (start 77.74 77.5) (end 78.5 77.5) (width 0.2) (layer "F.Cu") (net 11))
 (segment (start 77.12 58.5) (end 75.5 60.12) (width 0.2) (layer "F.Cu") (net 10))
 (segment (start 82.42 75.36) (end 82.42 58.985687) (width 0.2) (layer "F.Cu") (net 10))
 (segment (start 80.28 77.5) (end 82.42 75.36) (width 0.2) (layer "F.Cu") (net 10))
 (segment (start 81.934313 58.5) (end 77.12 58.5) (width 0.2) (layer "F.Cu") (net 10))
 (segment (start 82.42 58.985687) (end 81.934313 58.5) (width 0.2) (layer "F.Cu") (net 10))
 (segment (start 49.8 77.5) (end 44.860001 72.560001) (width 0.2) (layer "B.Cu") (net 22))
 (segment (start 44.860001 57.739999) (end 50.1 52.5) (width 0.2) (layer "B.Cu") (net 22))
 (segment (start 44.860001 72.560001) (end 44.860001 57.739999) (width 0.2) (layer "B.Cu") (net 22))
 (segment (start 74.98 58.1) (end 72.96 60.12) (width 0.2) (layer "F.Cu") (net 9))
 (segment (start 82.82 58.820001) (end 82.099998 58.1) (width 0.2) (layer "F.Cu") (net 9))
 (segment (start 82.099998 58.1) (end 74.98 58.1) (width 0.2) (layer "F.Cu") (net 9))
 (segment (start 82.82 77.5) (end 82.82 58.820001) (width 0.2) (layer "F.Cu") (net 9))
 (segment (start 48.14 57) (end 52.64 52.5) (width 0.2) (layer "B.Cu") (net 21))
 (segment (start 45.260001 58.522942) (end 46.782945 57) (width 0.2) (layer "B.Cu") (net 21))
 (segment (start 45.260001 70.420001) (end 45.260001 58.522942) (width 0.2) (layer "B.Cu") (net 21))
 (segment (start 46.782945 57) (end 48.14 57) (width 0.2) (layer "B.Cu") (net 21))
 (segment (start 52.34 77.5) (end 45.260001 70.420001) (width 0.2) (layer "B.Cu") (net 21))
 (segment (start 74.06 76.1) (end 74.06 59.02) (width 0.2) (layer "B.Cu") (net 13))
 (segment (start 72.66 77.5) (end 74.06 76.1) (width 0.2) (layer "B.Cu") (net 13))
 (segment (start 74.06 59.02) (end 80.58 52.5) (width 0.2) (layer "B.Cu") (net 13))
 (segment (start 66.78 75.76) (end 66.78 58.68) (width 0.2) (layer "B.Cu") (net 16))
 (segment (start 66.78 58.68) (end 72.96 52.5) (width 0.2) (layer "B.Cu") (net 16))
 (segment (start 65.04 77.5) (end 66.78 75.76) (width 0.2) (layer "B.Cu") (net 16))
 (segment (start 85.36 77.5) (end 83.22 75.36) (width 0.2) (layer "F.Cu") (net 8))
 (segment (start 82.265683 57.7) (end 62.68 57.7) (width 0.2) (layer "F.Cu") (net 8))
 (segment (start 83.22 58.654315) (end 82.265683 57.7) (width 0.2) (layer "F.Cu") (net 8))
 (segment (start 62.68 57.7) (end 60.26 60.12) (width 0.2) (layer "F.Cu") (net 8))
 (segment (start 83.22 75.36) (end 83.22 58.654315) (width 0.2) (layer "F.Cu") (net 8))
 (segment (start 46.46 59.02) (end 47.28 58.2) (width 0.2) (layer "B.Cu") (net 18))
 (segment (start 47.28 58.2) (end 54.56 58.2) (width 0.2) (layer "B.Cu") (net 18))
 (segment (start 54.56 58.2) (end 60.26 52.5) (width 0.2) (layer "B.Cu") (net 18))
 (segment (start 59.96 77.5) (end 46.46 64) (width 0.2) (layer "B.Cu") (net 18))
 (segment (start 46.46 64) (end 46.46 59.02) (width 0.2) (layer "B.Cu") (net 18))
 (segment (start 66.5 63.5) (end 66.5 61.5) (width 0.2) (layer "F.Cu") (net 26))
 (segment (start 66.5 61.5) (end 67.88 60.12) (width 0.2) (layer "F.Cu") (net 26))
 (segment (start 70.42 62.42) (end 70.42 60.12) (width 0.2) (layer "F.Cu") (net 27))
 (segment (start 71.5 63.5) (end 70.42 62.42) (width 0.2) (layer "F.Cu") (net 27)))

